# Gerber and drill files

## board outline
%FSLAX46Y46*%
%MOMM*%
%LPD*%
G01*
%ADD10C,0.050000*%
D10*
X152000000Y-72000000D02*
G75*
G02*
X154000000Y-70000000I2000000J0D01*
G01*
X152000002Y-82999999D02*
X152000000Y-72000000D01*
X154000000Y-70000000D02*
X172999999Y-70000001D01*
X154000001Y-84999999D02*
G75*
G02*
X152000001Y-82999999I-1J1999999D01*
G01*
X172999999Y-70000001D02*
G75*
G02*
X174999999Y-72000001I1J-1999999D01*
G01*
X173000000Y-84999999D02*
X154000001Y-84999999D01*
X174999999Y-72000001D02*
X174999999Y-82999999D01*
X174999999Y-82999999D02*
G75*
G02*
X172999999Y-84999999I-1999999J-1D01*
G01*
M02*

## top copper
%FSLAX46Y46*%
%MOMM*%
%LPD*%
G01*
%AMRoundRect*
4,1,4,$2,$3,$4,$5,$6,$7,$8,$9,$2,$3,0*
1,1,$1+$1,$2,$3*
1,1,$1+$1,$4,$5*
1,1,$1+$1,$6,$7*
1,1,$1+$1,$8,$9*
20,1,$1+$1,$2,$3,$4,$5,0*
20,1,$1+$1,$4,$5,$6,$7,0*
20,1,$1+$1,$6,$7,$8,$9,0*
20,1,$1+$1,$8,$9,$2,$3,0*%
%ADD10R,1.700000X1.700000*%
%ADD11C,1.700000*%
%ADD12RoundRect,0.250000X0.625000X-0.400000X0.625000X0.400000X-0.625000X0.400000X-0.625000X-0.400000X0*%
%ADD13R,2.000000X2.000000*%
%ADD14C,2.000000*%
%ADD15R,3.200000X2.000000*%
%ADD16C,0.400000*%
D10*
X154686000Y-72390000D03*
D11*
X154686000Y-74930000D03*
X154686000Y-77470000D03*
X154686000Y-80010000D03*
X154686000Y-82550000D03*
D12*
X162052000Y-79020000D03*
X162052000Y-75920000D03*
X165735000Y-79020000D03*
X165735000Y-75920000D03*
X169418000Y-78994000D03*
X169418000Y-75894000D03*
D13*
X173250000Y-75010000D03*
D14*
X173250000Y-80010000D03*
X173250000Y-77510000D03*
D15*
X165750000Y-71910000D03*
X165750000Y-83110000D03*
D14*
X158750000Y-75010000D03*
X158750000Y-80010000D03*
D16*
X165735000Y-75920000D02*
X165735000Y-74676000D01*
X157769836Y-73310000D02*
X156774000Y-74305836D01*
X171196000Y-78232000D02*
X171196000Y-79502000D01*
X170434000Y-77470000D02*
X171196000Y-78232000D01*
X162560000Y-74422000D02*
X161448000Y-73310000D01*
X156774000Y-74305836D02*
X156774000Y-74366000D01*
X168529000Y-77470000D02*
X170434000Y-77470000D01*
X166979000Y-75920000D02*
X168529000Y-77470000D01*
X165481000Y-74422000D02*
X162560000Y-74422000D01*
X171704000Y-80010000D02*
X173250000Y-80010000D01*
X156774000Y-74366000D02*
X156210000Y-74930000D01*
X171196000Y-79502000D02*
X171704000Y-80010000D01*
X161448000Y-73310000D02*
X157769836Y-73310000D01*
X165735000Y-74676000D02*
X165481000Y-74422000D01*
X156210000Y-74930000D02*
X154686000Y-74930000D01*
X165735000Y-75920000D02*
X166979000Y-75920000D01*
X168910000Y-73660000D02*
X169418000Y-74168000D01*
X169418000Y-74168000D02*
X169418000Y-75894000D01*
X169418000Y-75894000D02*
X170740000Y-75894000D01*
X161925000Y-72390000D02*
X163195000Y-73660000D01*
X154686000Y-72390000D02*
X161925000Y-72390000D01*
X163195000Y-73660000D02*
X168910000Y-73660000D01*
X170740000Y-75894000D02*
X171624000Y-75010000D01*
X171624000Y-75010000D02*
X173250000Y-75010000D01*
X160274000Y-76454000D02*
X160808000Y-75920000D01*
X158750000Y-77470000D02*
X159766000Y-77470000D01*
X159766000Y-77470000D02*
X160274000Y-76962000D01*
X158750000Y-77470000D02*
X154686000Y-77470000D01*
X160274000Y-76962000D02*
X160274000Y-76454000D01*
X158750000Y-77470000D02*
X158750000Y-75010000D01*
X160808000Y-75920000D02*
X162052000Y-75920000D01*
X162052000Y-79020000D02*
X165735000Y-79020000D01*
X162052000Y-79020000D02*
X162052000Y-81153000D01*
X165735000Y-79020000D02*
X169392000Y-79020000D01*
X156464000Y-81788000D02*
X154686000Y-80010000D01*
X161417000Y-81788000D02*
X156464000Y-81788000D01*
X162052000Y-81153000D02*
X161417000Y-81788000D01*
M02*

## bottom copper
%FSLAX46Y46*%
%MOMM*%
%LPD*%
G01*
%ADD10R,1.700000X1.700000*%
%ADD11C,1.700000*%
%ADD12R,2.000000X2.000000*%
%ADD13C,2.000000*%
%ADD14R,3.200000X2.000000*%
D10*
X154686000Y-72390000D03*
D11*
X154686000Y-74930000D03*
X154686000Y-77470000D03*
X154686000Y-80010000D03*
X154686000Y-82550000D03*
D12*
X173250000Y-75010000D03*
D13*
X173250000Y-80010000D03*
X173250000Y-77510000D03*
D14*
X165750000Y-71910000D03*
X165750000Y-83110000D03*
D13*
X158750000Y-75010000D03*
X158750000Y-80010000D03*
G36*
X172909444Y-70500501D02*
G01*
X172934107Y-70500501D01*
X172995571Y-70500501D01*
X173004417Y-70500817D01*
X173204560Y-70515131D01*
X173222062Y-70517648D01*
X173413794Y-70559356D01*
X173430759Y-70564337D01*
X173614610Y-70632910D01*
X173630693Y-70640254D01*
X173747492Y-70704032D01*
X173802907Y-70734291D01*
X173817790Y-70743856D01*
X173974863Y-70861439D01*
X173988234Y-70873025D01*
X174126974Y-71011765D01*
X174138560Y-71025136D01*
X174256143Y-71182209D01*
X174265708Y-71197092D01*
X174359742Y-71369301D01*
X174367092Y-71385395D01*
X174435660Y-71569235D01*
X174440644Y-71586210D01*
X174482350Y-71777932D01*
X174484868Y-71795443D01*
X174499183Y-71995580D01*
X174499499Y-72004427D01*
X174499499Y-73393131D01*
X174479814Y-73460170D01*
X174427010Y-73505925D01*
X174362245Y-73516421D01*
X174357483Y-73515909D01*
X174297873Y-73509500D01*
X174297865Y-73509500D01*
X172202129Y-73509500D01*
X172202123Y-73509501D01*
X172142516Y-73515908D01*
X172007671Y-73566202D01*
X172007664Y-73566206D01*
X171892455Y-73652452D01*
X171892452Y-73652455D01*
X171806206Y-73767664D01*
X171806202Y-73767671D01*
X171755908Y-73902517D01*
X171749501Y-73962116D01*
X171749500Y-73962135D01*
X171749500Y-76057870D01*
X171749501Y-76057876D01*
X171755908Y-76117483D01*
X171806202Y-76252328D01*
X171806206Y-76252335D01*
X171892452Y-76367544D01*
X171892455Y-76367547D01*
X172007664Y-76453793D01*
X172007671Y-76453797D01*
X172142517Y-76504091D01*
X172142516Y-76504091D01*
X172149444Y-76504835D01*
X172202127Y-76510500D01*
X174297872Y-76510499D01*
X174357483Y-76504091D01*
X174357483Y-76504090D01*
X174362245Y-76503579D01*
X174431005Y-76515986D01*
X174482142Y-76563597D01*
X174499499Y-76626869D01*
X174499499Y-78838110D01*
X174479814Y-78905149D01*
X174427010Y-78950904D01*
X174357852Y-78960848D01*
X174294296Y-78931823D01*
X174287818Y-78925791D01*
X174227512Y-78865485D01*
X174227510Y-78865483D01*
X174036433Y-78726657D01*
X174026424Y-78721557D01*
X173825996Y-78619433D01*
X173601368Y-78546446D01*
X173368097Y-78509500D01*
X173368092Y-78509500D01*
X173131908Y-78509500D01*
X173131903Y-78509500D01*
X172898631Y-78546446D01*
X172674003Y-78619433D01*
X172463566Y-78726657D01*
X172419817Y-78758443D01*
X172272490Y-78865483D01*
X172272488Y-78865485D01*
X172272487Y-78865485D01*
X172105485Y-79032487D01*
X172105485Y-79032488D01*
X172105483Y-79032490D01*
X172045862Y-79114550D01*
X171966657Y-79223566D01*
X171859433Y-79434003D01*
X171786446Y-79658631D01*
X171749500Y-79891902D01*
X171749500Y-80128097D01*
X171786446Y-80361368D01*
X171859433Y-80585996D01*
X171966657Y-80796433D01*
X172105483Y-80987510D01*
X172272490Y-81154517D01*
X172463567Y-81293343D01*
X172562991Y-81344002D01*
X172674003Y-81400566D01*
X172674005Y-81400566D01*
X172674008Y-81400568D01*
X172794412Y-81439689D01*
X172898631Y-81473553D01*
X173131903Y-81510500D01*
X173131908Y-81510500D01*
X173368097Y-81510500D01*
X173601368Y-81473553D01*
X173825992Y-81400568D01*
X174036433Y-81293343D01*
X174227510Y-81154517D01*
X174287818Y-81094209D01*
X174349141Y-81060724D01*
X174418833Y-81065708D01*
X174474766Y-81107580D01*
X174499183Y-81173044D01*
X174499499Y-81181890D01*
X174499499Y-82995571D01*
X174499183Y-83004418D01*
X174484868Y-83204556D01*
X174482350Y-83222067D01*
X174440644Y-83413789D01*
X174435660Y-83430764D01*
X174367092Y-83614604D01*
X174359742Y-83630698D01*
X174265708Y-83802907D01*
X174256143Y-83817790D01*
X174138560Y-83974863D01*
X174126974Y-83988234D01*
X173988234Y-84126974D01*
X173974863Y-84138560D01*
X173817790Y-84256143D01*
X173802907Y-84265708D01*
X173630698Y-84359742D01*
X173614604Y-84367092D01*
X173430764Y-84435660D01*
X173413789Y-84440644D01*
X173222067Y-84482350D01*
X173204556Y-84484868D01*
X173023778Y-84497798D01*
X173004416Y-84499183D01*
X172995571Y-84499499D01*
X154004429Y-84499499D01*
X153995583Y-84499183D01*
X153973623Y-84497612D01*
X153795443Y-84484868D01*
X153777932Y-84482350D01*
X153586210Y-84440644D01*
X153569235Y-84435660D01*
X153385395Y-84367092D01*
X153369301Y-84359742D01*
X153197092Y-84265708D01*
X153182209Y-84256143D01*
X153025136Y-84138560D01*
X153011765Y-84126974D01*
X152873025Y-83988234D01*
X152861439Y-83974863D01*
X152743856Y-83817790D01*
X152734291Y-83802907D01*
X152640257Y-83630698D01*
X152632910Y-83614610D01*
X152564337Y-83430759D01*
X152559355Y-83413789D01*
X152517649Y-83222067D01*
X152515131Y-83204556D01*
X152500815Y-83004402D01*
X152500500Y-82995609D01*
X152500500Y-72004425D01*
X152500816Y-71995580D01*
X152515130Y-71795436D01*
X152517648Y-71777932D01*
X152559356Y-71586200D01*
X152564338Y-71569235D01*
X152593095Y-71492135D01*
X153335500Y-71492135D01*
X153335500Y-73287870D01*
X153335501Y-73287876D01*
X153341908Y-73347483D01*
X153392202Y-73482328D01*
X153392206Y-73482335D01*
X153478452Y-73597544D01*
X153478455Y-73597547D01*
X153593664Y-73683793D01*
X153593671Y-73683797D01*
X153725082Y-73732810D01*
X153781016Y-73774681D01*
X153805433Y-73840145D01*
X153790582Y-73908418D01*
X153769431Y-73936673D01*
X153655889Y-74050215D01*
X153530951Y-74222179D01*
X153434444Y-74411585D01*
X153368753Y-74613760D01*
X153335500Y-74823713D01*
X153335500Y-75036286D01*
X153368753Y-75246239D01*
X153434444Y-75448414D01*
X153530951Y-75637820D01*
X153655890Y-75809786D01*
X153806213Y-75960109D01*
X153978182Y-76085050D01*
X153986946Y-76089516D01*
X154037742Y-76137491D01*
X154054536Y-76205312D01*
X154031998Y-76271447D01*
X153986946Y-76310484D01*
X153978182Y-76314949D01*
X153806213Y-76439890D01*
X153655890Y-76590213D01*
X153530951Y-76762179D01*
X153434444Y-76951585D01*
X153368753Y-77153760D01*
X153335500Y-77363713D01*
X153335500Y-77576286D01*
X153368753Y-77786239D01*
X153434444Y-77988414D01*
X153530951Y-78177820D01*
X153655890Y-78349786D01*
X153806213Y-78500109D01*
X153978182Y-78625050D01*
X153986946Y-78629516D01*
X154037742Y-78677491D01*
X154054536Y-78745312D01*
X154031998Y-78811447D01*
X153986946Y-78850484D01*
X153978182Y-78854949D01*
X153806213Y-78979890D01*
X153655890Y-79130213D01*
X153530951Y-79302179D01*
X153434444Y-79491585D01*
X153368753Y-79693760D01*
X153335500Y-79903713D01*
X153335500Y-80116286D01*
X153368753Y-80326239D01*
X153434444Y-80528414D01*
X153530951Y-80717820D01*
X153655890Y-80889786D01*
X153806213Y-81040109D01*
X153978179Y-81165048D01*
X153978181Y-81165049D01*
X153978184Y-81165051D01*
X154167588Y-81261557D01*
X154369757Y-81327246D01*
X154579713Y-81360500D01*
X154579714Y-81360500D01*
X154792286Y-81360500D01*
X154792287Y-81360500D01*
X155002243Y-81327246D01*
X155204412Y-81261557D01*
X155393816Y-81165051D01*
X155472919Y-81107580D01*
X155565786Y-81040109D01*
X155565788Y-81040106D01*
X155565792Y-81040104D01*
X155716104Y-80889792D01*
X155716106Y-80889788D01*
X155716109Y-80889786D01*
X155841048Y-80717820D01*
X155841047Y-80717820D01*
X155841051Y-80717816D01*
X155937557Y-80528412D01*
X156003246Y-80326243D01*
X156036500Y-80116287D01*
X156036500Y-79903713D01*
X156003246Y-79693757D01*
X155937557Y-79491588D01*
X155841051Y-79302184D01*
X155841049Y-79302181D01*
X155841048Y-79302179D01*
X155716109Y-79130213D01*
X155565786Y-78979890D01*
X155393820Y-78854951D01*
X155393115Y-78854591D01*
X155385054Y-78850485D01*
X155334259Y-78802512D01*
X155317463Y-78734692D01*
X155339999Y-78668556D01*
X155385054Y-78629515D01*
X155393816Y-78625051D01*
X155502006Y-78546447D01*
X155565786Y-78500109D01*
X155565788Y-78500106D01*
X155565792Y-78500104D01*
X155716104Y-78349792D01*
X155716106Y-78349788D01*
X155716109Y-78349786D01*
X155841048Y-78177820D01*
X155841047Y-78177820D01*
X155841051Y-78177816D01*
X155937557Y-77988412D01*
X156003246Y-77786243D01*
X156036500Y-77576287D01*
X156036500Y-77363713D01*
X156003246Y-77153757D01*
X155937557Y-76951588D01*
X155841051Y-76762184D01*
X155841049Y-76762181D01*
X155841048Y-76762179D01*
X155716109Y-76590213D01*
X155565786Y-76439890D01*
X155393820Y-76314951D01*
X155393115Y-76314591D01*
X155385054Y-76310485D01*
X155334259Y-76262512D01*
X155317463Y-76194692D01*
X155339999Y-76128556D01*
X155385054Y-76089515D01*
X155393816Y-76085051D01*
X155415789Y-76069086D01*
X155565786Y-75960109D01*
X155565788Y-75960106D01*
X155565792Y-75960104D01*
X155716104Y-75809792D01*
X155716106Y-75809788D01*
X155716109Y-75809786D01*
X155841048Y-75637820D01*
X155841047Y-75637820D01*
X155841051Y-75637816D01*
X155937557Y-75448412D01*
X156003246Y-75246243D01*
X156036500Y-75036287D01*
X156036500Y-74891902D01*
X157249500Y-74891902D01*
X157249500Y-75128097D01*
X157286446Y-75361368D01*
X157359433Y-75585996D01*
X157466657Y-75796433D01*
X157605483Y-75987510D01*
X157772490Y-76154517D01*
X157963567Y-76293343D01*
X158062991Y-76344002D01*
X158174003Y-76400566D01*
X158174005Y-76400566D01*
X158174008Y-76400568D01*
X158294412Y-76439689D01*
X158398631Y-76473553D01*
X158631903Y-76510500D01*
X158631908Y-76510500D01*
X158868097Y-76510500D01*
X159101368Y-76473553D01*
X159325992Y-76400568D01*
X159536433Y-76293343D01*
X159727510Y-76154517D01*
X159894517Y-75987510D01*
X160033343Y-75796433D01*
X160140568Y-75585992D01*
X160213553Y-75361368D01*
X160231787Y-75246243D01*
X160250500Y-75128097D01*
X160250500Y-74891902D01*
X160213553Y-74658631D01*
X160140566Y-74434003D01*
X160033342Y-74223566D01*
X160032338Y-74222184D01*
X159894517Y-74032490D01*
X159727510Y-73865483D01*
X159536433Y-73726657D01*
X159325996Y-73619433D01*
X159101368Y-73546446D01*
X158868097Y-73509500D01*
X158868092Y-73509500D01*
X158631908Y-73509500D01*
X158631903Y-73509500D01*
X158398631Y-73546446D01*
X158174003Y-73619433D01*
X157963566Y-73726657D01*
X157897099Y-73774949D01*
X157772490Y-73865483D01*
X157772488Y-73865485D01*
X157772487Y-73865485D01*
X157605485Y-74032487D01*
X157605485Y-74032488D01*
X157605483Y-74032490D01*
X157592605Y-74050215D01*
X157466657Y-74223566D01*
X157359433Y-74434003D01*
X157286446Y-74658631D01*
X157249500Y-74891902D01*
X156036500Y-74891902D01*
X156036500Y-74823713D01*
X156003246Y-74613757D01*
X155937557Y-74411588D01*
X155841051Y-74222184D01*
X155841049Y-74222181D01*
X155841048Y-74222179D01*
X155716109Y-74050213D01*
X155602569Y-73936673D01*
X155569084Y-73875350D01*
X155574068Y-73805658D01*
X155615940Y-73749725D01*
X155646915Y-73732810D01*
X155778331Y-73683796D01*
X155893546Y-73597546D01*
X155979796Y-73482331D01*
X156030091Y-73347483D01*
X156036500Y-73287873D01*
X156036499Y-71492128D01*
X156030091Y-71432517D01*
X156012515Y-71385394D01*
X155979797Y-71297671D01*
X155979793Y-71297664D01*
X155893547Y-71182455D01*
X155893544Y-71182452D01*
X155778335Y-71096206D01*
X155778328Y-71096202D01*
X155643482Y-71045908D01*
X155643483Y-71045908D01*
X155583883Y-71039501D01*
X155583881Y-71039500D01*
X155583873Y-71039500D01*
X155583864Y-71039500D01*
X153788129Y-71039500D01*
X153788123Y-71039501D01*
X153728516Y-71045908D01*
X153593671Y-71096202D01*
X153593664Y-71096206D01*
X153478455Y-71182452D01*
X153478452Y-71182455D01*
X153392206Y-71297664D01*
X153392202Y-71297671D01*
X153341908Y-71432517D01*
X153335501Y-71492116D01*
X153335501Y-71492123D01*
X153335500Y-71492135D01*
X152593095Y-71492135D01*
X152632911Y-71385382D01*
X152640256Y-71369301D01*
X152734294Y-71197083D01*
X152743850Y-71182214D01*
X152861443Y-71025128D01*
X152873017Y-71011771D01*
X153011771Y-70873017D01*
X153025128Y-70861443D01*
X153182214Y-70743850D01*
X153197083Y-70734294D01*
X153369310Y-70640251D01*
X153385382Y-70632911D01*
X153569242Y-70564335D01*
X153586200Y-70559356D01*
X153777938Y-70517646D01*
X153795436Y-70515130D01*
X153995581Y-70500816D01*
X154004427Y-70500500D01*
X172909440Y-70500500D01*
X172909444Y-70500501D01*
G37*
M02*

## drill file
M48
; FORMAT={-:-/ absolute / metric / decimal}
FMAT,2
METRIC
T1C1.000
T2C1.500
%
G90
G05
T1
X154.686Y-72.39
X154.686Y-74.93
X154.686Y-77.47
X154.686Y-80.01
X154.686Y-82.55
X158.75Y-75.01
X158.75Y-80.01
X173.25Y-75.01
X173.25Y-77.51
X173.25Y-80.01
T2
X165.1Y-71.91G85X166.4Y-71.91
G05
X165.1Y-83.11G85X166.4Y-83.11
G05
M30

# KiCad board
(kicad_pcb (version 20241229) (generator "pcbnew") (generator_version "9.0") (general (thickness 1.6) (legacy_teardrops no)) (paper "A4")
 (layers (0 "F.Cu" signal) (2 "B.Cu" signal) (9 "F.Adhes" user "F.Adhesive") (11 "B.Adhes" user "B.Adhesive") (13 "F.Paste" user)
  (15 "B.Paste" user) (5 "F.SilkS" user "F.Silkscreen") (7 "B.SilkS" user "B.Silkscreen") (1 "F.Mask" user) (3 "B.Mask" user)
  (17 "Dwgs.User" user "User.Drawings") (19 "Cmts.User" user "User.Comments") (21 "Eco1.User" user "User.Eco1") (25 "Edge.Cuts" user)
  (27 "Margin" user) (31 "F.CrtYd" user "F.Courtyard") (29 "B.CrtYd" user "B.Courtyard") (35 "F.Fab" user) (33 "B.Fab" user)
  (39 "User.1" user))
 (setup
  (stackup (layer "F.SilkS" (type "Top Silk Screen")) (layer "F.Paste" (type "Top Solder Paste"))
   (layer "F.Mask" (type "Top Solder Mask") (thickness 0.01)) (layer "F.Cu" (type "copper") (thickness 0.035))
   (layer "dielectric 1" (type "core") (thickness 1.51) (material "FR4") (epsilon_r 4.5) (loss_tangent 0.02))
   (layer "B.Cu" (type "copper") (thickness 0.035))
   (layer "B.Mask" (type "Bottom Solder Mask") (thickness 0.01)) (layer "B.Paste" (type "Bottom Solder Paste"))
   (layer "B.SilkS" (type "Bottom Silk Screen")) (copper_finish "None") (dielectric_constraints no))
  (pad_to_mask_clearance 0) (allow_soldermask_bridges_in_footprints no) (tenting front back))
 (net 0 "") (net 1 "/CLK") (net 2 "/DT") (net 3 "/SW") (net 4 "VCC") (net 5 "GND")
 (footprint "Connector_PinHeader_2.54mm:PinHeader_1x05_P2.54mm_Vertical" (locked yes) (layer "F.Cu") (at 154.686 72.39)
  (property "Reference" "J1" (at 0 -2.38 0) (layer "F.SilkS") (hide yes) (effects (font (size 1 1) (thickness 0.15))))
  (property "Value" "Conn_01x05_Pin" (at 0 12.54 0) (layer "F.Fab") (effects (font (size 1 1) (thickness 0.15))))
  (pad "1" thru_hole rect (at 0 0) (size 1.7 1.7) (drill 1) (layers "*.Cu" "*.Mask") (remove_unused_layers no) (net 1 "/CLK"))
  (pad "2" thru_hole circle (at 0 2.54) (size 1.7 1.7) (drill 1) (layers "*.Cu" "*.Mask") (remove_unused_layers no) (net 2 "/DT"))
  (pad "3" thru_hole circle (at 0 5.08) (size 1.7 1.7) (drill 1) (layers "*.Cu" "*.Mask") (remove_unused_layers no) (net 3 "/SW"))
  (pad "4" thru_hole circle (at 0 7.62) (size 1.7 1.7) (drill 1) (layers "*.Cu" "*.Mask") (remove_unused_layers no) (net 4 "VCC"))
  (pad "5" thru_hole circle (at 0 10.16) (size 1.7 1.7) (drill 1) (layers "*.Cu" "*.Mask") (remove_unused_layers no) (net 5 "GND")))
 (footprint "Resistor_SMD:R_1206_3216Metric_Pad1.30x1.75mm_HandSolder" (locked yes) (layer "F.Cu") (at 162.052 77.47 90)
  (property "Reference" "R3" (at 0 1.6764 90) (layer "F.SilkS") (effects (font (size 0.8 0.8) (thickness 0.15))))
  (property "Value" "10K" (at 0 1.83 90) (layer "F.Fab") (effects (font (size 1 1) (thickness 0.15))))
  (pad "1" smd roundrect (at -1.55 0 90) (size 1.3 1.75) (layers "F.Cu" "F.Mask" "F.Paste") (roundrect_rratio 0.192308) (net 4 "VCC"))
  (pad "2" smd roundrect (at 1.55 0 90) (size 1.3 1.75) (layers "F.Cu" "F.Mask" "F.Paste") (roundrect_rratio 0.192308) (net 3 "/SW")))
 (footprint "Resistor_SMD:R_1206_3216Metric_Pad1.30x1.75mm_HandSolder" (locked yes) (layer "F.Cu") (at 165.735 77.47 90)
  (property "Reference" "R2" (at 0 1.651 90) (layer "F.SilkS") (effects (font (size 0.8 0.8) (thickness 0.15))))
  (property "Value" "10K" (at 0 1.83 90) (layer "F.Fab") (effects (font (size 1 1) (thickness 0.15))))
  (pad "1" smd roundrect (at -1.55 0 90) (size 1.3 1.75) (layers "F.Cu" "F.Mask" "F.Paste") (roundrect_rratio 0.192308) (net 4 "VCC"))
  (pad "2" smd roundrect (at 1.55 0 90) (size 1.3 1.75) (layers "F.Cu" "F.Mask" "F.Paste") (roundrect_rratio 0.192308) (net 2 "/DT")))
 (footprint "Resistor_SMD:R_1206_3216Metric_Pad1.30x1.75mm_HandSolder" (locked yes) (layer "F.Cu") (at 169.418 77.444 90)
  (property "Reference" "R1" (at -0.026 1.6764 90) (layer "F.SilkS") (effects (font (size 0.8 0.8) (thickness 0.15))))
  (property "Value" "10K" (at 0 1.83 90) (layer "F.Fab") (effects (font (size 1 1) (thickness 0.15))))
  (pad "1" smd roundrect (at -1.55 0 90) (size 1.3 1.75) (layers "F.Cu" "F.Mask" "F.Paste") (roundrect_rratio 0.192308) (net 4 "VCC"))
  (pad "2" smd roundrect (at 1.55 0 90) (size 1.3 1.75) (layers "F.Cu" "F.Mask" "F.Paste") (roundrect_rratio 0.192308) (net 1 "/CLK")))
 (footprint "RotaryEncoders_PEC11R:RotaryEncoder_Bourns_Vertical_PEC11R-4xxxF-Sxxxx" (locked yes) (layer "B.Cu") (at 165.75 77.51 -90)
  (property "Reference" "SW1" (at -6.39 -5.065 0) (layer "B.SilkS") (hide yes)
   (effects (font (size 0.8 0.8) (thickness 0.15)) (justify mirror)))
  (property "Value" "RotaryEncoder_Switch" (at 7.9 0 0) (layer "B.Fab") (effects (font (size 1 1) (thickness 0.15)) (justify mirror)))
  (pad "A" thru_hole rect (at -2.5 -7.5 180) (size 2 2) (drill 1) (layers "*.Cu" "*.Mask") (remove_unused_layers no) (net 1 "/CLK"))
  (pad "B" thru_hole circle (at 2.5 -7.5 180) (size 2 2) (drill 1) (layers "*.Cu" "*.Mask") (remove_unused_layers no) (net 2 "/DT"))
  (pad "C" thru_hole circle (at 0 -7.5 180) (size 2 2) (drill 1) (layers "*.Cu" "*.Mask") (remove_unused_layers no) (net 5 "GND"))
  (pad "MP" thru_hole rect (at -5.6 0) (size 3.2 2) (drill oval 2.8 1.5) (layers "*.Cu" "*.Mask") (remove_unused_layers no) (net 5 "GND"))
  (pad "MP" thru_hole rect (at 5.6 0) (size 3.2 2) (drill oval 2.8 1.5) (layers "*.Cu" "*.Mask") (remove_unused_layers no) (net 5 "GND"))
  (pad "S1" thru_hole circle (at -2.5 7) (size 2 2) (drill 1) (layers "*.Cu" "*.Mask") (remove_unused_layers no) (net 3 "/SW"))
  (pad "S2" thru_hole circle (at 2.5 7) (size 2 2) (drill 1) (layers "*.Cu" "*.Mask") (remove_unused_layers no) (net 5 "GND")))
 (gr_arc (start 152 72) (mid 152.585786 70.585786) (end 154 70) (stroke (width 0.05) (type default)) (layer "Edge.Cuts"))
 (gr_line (start 152.000002 82.999999) (end 152 72) (stroke (width 0.05) (type default)) (layer "Edge.Cuts"))
 (gr_line (start 154 70) (end 172.999999 70.000001) (stroke (width 0.05) (type default)) (layer "Edge.Cuts"))
 (gr_arc (start 154.000001 84.999999) (mid 152.585787 84.414213) (end 152.000001 82.999999) (stroke (width 0.05) (type default))
  (layer "Edge.Cuts"))
 (gr_arc (start 172.999999 70.000001) (mid 174.414213 70.585787) (end 174.999999 72.000001) (stroke (width 0.05) (type default))
  (layer "Edge.Cuts"))
 (gr_line (start 173 84.999999) (end 154.000001 84.999999) (stroke (width 0.05) (type default)) (layer "Edge.Cuts"))
 (gr_line (start 174.999999 72.000001) (end 174.999999 82.999999) (stroke (width 0.05) (type default)) (layer "Edge.Cuts"))
 (gr_arc (start 174.999999 82.999999) (mid 174.414213 84.414213) (end 172.999999 84.999999) (stroke (width 0.05) (type default))
  (layer "Edge.Cuts"))
 (segment (start 165.735 75.92) (end 165.735 74.676) (width 0.4) (layer "F.Cu") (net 2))
 (segment (start 157.769836 73.31) (end 156.774 74.305836) (width 0.4) (layer "F.Cu") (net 2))
 (segment (start 171.196 78.232) (end 171.196 79.502) (width 0.4) (layer "F.Cu") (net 2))
 (segment (start 170.434 77.47) (end 171.196 78.232) (width 0.4) (layer "F.Cu") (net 2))
 (segment (start 162.56 74.422) (end 161.448 73.31) (width 0.4) (layer "F.Cu") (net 2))
 (segment (start 156.774 74.305836) (end 156.774 74.366) (width 0.4) (layer "F.Cu") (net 2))
 (segment (start 168.529 77.47) (end 170.434 77.47) (width 0.4) (layer "F.Cu") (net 2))
 (segment (start 166.979 75.92) (end 168.529 77.47) (width 0.4) (layer "F.Cu") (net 2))
 (segment (start 165.481 74.422) (end 162.56 74.422) (width 0.4) (layer "F.Cu") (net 2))
 (segment (start 171.704 80.01) (end 173.25 80.01) (width 0.4) (layer "F.Cu") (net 2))
 (segment (start 156.774 74.366) (end 156.21 74.93) (width 0.4) (layer "F.Cu") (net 2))
 (segment (start 171.196 79.502) (end 171.704 80.01) (width 0.4) (layer "F.Cu") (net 2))
 (segment (start 161.448 73.31) (end 157.769836 73.31) (width 0.4) (layer "F.Cu") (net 2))
 (segment (start 165.735 74.676) (end 165.481 74.422) (width 0.4) (layer "F.Cu") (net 2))
 (segment (start 156.21 74.93) (end 154.686 74.93) (width 0.4) (layer "F.Cu") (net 2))
 (segment (start 165.735 75.92) (end 166.979 75.92) (width 0.4) (layer "F.Cu") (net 2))
 (segment (start 168.91 73.66) (end 169.418 74.168) (width 0.4) (layer "F.Cu") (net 1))
 (segment (start 169.418 74.168) (end 169.418 75.894) (width 0.4) (layer "F.Cu") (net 1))
 (segment (start 169.418 75.894) (end 170.74 75.894) (width 0.4) (layer "F.Cu") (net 1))
 (segment (start 161.925 72.39) (end 163.195 73.66) (width 0.4) (layer "F.Cu") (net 1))
 (segment (start 154.686 72.39) (end 161.925 72.39) (width 0.4) (layer "F.Cu") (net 1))
 (segment (start 163.195 73.66) (end 168.91 73.66) (width 0.4) (layer "F.Cu") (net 1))
 (segment (start 170.74 75.894) (end 171.624 75.01) (width 0.4) (layer "F.Cu") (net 1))
 (segment (start 171.624 75.01) (end 173.25 75.01) (width 0.4) (layer "F.Cu") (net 1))
 (segment (start 160.274 76.454) (end 160.808 75.92) (width 0.4) (layer "F.Cu") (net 3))
 (segment (start 158.75 77.47) (end 159.766 77.47) (width 0.4) (layer "F.Cu") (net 3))
 (segment (start 159.766 77.47) (end 160.274 76.962) (width 0.4) (layer "F.Cu") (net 3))
 (segment (start 158.75 77.47) (end 154.686 77.47) (width 0.4) (layer "F.Cu") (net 3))
 (segment (start 160.274 76.962) (end 160.274 76.454) (width 0.4) (layer "F.Cu") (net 3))
 (segment (start 158.75 77.47) (end 158.75 75.01) (width 0.4) (layer "F.Cu") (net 3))
 (segment (start 160.808 75.92) (end 162.052 75.92) (width 0.4) (layer "F.Cu") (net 3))
 (segment (start 162.052 79.02) (end 165.735 79.02) (width 0.4) (layer "F.Cu") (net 4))
 (segment (start 162.052 79.02) (end 162.052 81.153) (width 0.4) (layer "F.Cu") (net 4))
 (segment (start 165.735 79.02) (end 169.392 79.02) (width 0.4) (layer "F.Cu") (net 4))
 (segment (start 156.464 81.788) (end 154.686 80.01) (width 0.4) (layer "F.Cu") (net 4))
 (segment (start 161.417 81.788) (end 156.464 81.788) (width 0.4) (layer "F.Cu") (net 4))
 (segment (start 162.052 81.153) (end 161.417 81.788) (width 0.4) (layer "F.Cu") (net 4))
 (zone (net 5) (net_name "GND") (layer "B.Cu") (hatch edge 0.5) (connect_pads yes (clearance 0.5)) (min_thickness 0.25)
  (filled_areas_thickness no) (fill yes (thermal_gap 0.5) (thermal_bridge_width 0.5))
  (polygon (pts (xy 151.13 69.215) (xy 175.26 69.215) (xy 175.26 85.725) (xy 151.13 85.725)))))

